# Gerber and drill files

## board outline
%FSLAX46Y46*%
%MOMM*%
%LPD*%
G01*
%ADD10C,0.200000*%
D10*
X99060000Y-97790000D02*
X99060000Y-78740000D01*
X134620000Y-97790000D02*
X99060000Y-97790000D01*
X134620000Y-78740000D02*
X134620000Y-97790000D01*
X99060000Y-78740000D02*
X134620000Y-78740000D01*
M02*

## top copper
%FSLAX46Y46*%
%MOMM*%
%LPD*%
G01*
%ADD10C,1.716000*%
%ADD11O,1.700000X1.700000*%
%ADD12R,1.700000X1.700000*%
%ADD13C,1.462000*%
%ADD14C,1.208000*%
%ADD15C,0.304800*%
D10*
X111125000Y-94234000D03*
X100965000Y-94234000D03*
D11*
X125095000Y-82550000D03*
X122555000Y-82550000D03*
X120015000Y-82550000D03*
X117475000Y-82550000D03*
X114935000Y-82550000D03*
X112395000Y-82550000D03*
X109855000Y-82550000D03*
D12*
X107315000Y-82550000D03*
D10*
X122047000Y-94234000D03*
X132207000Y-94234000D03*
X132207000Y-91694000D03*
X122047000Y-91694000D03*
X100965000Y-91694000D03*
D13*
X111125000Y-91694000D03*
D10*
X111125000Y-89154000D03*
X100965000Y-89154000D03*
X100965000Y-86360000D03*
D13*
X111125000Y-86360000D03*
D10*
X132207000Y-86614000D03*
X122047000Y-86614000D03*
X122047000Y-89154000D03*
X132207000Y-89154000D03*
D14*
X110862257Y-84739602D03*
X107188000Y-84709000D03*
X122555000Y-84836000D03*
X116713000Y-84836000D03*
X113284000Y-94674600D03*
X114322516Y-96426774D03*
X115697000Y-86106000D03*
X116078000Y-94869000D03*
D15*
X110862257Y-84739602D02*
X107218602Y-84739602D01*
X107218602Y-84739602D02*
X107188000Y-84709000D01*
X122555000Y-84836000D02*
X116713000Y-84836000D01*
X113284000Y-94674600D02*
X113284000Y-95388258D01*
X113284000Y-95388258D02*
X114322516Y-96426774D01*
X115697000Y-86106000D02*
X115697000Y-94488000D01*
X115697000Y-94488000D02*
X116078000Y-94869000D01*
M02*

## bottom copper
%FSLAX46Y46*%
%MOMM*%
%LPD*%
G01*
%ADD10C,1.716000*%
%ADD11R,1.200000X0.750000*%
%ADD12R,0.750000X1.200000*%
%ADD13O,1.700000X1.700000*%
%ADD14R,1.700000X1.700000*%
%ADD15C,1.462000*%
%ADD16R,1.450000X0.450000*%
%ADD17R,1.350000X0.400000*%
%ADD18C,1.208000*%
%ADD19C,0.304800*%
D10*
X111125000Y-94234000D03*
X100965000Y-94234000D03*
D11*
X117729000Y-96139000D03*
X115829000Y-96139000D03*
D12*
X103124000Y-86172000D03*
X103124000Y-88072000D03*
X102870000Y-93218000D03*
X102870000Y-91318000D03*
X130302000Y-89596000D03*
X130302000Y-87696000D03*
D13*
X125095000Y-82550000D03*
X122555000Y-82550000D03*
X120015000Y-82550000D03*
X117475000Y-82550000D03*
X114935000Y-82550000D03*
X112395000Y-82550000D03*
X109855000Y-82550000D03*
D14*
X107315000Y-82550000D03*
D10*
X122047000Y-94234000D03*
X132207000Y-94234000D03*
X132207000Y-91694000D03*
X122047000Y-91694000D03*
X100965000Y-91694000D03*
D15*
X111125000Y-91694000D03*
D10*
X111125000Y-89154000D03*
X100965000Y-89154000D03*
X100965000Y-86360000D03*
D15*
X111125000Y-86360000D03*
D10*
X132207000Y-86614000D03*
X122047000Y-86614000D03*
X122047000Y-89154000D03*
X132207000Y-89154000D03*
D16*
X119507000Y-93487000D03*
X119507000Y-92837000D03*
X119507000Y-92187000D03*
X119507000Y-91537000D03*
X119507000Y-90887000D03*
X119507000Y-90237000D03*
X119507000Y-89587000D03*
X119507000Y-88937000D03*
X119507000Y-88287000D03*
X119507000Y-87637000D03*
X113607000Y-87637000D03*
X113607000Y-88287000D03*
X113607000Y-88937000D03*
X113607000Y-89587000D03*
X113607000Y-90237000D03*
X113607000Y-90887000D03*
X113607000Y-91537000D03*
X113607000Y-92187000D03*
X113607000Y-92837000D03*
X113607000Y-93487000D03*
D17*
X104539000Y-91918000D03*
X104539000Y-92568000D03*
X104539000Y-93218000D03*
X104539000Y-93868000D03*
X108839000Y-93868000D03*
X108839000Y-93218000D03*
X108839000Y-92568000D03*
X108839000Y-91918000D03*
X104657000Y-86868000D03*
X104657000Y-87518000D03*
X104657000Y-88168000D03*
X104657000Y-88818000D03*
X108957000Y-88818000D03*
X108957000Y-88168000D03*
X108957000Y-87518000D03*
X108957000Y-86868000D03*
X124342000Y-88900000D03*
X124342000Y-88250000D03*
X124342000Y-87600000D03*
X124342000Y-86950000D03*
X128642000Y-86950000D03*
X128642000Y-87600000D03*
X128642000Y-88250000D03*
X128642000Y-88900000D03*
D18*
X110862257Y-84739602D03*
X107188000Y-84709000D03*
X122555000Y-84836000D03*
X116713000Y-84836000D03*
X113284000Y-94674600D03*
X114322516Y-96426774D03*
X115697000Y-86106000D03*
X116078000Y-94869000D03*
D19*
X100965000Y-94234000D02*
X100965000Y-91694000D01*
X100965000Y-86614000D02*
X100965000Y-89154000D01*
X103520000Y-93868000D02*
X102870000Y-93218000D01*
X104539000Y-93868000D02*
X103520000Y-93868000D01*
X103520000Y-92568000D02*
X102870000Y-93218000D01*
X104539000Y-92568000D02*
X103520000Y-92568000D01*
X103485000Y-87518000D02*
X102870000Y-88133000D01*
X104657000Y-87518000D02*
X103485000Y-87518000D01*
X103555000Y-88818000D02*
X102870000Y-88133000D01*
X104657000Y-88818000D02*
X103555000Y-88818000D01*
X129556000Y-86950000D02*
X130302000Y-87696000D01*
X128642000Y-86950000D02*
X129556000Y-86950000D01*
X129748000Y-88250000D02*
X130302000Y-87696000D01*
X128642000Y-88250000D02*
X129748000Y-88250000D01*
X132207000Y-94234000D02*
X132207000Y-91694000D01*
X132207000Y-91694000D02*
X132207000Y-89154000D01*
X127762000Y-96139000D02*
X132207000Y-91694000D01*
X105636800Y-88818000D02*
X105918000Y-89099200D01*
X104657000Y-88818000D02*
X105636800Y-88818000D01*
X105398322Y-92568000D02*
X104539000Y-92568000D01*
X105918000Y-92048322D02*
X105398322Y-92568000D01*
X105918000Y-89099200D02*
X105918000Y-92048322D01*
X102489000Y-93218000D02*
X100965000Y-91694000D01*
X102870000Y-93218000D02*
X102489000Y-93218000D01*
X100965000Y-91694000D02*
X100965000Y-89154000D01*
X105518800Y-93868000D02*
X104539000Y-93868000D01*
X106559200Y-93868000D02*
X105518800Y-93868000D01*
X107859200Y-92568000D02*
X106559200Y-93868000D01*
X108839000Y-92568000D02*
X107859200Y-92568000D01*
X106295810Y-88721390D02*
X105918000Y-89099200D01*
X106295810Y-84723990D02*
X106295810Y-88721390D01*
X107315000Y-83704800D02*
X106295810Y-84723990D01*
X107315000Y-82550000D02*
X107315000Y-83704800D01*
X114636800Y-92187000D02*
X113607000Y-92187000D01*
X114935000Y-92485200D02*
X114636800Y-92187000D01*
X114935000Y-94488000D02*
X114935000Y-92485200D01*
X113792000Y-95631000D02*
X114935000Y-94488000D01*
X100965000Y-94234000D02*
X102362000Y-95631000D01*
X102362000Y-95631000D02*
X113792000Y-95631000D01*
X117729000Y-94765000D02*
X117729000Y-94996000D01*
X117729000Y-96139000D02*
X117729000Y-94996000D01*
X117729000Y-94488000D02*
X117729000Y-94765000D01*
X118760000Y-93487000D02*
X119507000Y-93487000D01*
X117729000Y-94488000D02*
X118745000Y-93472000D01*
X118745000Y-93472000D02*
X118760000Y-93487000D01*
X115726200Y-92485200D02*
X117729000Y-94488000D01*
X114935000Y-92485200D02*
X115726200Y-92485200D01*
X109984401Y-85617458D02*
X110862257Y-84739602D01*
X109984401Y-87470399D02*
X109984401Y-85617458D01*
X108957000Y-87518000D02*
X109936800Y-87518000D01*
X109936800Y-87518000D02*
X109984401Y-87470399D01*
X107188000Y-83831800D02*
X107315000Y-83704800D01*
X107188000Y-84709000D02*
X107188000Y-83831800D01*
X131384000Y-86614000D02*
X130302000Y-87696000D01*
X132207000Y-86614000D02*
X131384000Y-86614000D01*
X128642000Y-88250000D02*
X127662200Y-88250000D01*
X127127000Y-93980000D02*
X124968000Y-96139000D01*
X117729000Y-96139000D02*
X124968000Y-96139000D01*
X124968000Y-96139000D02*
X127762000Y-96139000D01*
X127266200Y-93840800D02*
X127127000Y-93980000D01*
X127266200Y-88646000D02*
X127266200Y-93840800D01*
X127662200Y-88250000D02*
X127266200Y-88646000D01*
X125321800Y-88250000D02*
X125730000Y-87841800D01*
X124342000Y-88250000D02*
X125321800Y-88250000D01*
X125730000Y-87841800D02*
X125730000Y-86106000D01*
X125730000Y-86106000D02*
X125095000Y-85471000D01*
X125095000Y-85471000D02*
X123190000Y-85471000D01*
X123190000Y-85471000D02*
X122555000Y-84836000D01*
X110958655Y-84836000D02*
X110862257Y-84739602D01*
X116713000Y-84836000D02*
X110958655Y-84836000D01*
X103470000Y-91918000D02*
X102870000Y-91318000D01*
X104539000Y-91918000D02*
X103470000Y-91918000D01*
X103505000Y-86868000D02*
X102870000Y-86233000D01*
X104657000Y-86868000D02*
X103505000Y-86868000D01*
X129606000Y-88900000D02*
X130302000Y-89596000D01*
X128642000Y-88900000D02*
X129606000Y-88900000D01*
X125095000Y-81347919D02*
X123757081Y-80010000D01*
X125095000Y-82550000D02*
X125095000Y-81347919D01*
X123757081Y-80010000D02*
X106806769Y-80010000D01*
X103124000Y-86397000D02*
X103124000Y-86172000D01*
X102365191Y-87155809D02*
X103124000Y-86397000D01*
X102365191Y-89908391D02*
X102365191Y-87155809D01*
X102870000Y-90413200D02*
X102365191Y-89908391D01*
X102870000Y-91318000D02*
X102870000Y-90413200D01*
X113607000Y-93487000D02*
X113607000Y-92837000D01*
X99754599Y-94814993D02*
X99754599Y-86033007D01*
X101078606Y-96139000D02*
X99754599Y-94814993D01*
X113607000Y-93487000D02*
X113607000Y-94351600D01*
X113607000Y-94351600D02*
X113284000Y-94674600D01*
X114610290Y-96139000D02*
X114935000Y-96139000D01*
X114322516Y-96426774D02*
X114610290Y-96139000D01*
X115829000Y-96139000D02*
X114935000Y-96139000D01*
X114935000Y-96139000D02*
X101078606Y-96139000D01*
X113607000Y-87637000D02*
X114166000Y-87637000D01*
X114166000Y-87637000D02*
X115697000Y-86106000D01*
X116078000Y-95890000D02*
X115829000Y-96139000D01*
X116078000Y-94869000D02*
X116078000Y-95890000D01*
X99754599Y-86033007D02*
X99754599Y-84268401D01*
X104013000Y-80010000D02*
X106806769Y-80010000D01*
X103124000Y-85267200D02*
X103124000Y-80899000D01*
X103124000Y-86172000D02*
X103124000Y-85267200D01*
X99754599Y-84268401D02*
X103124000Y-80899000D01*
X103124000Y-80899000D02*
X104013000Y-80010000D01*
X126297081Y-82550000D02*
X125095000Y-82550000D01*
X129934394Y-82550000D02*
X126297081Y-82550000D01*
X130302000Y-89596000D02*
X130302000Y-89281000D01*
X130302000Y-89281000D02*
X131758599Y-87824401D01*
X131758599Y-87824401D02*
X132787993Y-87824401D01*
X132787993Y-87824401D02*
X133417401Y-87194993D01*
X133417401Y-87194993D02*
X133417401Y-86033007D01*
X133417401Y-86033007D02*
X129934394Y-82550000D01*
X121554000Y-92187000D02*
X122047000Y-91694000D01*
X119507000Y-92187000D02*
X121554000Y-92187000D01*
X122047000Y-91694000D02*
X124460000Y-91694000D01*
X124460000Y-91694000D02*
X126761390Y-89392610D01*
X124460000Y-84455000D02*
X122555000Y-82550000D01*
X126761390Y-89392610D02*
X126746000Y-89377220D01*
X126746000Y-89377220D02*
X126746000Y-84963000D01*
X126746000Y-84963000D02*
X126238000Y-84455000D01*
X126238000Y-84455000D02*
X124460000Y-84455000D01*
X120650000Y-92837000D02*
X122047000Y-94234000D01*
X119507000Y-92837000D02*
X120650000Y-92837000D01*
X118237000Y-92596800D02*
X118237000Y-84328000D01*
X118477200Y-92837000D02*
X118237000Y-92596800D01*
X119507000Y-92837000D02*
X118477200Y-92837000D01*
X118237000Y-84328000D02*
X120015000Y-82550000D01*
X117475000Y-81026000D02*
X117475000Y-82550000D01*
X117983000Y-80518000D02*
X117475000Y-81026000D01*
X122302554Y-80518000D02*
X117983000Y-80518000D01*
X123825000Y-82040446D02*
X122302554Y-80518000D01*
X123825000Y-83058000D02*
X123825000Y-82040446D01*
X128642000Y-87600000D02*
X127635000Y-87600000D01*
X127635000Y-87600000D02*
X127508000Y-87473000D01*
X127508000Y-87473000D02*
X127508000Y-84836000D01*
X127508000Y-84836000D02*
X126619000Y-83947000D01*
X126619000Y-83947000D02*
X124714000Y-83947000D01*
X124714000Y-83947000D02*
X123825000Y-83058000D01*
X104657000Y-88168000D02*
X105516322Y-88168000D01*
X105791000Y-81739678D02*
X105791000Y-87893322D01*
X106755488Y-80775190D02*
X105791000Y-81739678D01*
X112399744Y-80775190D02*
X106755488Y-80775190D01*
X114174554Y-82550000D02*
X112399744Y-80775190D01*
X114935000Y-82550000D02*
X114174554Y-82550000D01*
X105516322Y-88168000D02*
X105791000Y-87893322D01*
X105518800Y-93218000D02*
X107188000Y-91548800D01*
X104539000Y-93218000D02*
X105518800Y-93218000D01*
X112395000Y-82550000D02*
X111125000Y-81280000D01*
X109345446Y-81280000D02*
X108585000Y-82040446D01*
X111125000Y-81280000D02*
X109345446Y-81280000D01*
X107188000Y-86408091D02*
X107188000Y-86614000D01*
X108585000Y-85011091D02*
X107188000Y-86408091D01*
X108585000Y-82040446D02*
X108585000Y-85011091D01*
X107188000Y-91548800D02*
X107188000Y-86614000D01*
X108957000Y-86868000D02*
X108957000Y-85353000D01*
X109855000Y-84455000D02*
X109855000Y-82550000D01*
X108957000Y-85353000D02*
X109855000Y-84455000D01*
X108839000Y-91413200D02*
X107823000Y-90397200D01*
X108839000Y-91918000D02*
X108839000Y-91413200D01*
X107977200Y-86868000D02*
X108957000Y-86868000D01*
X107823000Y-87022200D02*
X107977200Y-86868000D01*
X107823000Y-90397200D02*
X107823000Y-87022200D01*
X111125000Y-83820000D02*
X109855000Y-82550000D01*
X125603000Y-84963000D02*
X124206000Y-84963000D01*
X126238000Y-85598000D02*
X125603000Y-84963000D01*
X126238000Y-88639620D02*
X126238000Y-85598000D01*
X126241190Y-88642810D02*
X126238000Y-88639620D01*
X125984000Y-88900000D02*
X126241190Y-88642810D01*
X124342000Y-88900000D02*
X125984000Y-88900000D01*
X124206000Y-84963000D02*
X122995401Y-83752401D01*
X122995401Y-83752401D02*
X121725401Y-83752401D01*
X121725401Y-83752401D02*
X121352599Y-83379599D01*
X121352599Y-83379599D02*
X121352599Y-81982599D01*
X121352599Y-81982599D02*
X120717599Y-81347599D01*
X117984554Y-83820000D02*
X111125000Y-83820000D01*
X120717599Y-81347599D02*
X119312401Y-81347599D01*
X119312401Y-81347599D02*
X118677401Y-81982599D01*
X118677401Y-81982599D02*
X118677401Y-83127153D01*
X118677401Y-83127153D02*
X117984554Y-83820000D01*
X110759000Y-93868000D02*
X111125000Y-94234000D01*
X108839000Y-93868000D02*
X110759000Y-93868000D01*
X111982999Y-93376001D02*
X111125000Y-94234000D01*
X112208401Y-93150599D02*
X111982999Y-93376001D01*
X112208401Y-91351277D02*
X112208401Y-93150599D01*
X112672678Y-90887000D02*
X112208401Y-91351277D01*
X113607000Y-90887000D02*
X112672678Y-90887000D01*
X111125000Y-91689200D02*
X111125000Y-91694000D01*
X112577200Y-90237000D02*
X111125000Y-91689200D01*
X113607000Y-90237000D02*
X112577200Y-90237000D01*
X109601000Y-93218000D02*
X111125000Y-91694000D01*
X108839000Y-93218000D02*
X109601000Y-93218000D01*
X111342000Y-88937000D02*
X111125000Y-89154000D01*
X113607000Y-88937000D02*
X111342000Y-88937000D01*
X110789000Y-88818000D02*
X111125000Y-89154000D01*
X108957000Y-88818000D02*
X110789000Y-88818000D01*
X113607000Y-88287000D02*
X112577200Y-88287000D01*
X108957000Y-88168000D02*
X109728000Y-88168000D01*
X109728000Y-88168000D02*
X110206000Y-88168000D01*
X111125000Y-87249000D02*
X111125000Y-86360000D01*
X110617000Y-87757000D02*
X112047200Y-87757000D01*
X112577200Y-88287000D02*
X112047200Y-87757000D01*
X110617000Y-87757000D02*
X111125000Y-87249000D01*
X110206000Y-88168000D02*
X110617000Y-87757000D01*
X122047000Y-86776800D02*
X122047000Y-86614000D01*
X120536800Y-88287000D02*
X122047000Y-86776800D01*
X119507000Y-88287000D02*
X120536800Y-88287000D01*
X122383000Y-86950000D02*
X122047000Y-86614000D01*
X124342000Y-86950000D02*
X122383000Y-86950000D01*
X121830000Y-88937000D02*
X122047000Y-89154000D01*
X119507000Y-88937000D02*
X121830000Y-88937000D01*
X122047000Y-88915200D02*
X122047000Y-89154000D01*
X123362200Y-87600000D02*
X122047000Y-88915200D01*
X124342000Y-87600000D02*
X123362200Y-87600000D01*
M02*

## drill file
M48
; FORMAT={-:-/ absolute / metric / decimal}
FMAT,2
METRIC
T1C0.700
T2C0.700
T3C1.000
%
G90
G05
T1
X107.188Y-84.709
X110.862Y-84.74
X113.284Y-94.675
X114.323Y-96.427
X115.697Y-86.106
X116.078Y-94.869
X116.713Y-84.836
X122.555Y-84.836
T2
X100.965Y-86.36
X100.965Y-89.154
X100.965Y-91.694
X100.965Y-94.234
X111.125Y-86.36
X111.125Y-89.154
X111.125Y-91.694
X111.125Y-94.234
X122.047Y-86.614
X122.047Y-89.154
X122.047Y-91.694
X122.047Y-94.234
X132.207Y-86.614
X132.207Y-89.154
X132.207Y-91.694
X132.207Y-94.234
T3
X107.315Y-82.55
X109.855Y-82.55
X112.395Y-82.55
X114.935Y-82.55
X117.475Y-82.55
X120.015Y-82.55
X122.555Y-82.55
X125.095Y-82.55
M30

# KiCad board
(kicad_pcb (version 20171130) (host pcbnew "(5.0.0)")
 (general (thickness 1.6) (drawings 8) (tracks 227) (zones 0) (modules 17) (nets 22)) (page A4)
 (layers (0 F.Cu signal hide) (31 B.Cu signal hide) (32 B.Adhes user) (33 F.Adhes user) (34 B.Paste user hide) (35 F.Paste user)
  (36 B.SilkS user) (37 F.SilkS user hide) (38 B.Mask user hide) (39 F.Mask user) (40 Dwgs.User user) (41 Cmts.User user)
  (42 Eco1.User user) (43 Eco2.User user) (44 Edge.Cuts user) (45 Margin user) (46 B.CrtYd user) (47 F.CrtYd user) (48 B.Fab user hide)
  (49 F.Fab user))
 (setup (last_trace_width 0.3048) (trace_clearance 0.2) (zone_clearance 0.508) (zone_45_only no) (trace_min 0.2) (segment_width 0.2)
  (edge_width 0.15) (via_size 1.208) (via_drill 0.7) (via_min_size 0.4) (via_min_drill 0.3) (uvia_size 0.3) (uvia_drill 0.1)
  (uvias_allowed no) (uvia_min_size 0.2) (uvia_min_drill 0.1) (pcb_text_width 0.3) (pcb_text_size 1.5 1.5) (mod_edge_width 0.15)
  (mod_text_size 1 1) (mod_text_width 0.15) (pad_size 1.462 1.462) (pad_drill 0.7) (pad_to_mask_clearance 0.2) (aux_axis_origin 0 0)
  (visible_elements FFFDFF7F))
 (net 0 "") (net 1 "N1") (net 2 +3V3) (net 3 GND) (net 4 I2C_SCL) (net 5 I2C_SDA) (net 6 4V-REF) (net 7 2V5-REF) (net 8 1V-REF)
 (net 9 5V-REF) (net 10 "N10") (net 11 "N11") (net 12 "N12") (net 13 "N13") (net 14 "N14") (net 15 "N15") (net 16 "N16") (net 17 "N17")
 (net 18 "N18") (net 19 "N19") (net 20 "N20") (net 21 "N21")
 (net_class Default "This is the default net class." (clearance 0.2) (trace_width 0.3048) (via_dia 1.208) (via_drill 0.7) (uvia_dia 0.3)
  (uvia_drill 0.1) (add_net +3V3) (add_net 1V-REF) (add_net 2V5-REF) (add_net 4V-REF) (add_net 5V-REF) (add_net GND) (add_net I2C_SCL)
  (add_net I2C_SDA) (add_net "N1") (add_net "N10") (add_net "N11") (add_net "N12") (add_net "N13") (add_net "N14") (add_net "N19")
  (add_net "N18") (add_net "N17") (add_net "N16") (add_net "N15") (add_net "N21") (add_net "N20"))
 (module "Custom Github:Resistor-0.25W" (layer F.Cu) (at 100.965 94.234)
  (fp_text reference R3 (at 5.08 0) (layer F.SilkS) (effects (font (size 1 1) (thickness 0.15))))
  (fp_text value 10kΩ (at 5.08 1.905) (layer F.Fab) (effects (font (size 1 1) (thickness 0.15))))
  (pad 2 thru_hole circle (at 10.16 0) (size 1.716 1.716) (drill 0.7) (layers *.Cu *.Mask F.SilkS) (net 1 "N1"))
  (pad 1 thru_hole circle (at 0 0) (size 1.716 1.716) (drill 0.7) (layers *.Cu *.Mask F.SilkS) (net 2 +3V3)))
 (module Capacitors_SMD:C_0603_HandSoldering (layer B.Cu) (at 116.779 96.139 180)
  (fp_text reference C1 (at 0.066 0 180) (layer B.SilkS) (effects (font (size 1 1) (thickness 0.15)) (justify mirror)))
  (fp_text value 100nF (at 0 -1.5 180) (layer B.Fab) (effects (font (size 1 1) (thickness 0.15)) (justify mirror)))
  (pad 1 smd rect (at -0.95 0 180) (size 1.2 0.75) (layers B.Cu B.Paste B.Mask) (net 2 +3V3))
  (pad 2 smd rect (at 0.95 0 180) (size 1.2 0.75) (layers B.Cu B.Paste B.Mask) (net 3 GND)))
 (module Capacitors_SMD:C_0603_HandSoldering (layer B.Cu) (at 103.124 87.122 90)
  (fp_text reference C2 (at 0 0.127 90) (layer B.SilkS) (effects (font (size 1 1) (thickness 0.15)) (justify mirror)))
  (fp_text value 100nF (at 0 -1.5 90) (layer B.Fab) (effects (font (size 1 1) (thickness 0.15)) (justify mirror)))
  (pad 2 smd rect (at 0.95 0 90) (size 1.2 0.75) (layers B.Cu B.Paste B.Mask) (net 3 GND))
  (pad 1 smd rect (at -0.95 0 90) (size 1.2 0.75) (layers B.Cu B.Paste B.Mask) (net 2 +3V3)))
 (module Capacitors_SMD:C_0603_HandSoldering (layer B.Cu) (at 102.87 92.268 90)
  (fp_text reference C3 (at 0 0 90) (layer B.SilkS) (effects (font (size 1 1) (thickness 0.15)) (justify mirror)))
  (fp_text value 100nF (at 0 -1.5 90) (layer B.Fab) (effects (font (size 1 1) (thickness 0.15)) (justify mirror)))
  (pad 1 smd rect (at -0.95 0 90) (size 1.2 0.75) (layers B.Cu B.Paste B.Mask) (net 2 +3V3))
  (pad 2 smd rect (at 0.95 0 90) (size 1.2 0.75) (layers B.Cu B.Paste B.Mask) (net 3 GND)))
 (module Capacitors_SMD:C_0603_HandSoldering (layer B.Cu) (at 130.302 88.646 270)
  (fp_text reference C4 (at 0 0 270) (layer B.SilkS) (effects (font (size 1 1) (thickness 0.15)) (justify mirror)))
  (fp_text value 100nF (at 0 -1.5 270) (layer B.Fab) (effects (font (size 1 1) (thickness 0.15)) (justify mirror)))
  (pad 2 smd rect (at 0.95 0 270) (size 1.2 0.75) (layers B.Cu B.Paste B.Mask) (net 3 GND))
  (pad 1 smd rect (at -0.95 0 270) (size 1.2 0.75) (layers B.Cu B.Paste B.Mask) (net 2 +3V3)))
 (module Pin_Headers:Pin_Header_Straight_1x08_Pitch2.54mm (layer F.Cu) (at 107.315 82.55 90)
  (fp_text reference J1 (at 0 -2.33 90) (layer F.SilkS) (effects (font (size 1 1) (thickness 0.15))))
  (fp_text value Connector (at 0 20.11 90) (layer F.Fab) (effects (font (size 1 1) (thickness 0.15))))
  (pad 8 thru_hole oval (at 0 17.78 90) (size 1.7 1.7) (drill 1) (layers *.Cu *.Mask) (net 3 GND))
  (pad 7 thru_hole oval (at 0 15.24 90) (size 1.7 1.7) (drill 1) (layers *.Cu *.Mask) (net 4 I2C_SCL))
  (pad 6 thru_hole oval (at 0 12.7 90) (size 1.7 1.7) (drill 1) (layers *.Cu *.Mask) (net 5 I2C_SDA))
  (pad 5 thru_hole oval (at 0 10.16 90) (size 1.7 1.7) (drill 1) (layers *.Cu *.Mask) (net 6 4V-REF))
  (pad 4 thru_hole oval (at 0 7.62 90) (size 1.7 1.7) (drill 1) (layers *.Cu *.Mask) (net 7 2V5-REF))
  (pad 3 thru_hole oval (at 0 5.08 90) (size 1.7 1.7) (drill 1) (layers *.Cu *.Mask) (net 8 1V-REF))
  (pad 2 thru_hole oval (at 0 2.54 90) (size 1.7 1.7) (drill 1) (layers *.Cu *.Mask) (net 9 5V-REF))
  (pad 1 thru_hole rect (at 0 0 90) (size 1.7 1.7) (drill 1) (layers *.Cu *.Mask) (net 2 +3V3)))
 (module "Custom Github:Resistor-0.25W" (layer F.Cu) (at 132.207 94.234 180)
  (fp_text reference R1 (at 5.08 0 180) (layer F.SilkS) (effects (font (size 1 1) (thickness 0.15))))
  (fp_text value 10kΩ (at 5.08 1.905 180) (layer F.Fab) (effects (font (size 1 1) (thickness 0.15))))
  (pad 2 thru_hole circle (at 10.16 0 180) (size 1.716 1.716) (drill 0.7) (layers *.Cu *.Mask F.SilkS) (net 5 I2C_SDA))
  (pad 1 thru_hole circle (at 0 0 180) (size 1.716 1.716) (drill 0.7) (layers *.Cu *.Mask F.SilkS) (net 2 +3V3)))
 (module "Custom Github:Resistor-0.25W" (layer F.Cu) (at 132.207 91.694 180)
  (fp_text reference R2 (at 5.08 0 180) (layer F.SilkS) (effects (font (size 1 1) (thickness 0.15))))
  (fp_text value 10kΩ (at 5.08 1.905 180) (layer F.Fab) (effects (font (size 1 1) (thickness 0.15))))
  (pad 1 thru_hole circle (at 0 0 180) (size 1.716 1.716) (drill 0.7) (layers *.Cu *.Mask F.SilkS) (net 2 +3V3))
  (pad 2 thru_hole circle (at 10.16 0 180) (size 1.716 1.716) (drill 0.7) (layers *.Cu *.Mask F.SilkS) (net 4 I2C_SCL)))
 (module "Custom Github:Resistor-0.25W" (layer F.Cu) (at 100.965 91.694)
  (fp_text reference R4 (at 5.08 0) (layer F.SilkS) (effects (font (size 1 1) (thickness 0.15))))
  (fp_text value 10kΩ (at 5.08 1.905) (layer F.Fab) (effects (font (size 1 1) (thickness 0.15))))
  (pad 1 thru_hole circle (at 0 0) (size 1.716 1.716) (drill 0.7) (layers *.Cu *.Mask F.SilkS) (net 2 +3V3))
  (pad 2 thru_hole circle (at 10.16 0) (size 1.462 1.462) (drill 0.7) (layers *.Cu *.Mask F.SilkS) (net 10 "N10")))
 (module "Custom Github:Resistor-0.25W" (layer F.Cu) (at 100.965 89.154)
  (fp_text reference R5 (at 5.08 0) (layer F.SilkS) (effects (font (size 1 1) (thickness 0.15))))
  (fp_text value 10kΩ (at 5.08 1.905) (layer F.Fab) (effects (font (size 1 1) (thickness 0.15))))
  (pad 2 thru_hole circle (at 10.16 0) (size 1.716 1.716) (drill 0.7) (layers *.Cu *.Mask F.SilkS) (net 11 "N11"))
  (pad 1 thru_hole circle (at 0 0) (size 1.716 1.716) (drill 0.7) (layers *.Cu *.Mask F.SilkS) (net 2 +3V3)))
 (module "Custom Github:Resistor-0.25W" (layer F.Cu) (at 100.965 86.36)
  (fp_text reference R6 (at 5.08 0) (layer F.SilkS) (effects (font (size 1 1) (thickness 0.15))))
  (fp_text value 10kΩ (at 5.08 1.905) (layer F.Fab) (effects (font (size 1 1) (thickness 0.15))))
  (pad 1 thru_hole circle (at 0 0) (size 1.716 1.716) (drill 0.7) (layers *.Cu *.Mask F.SilkS) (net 2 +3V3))
  (pad 2 thru_hole circle (at 10.16 0) (size 1.462 1.462) (drill 0.7) (layers *.Cu *.Mask F.SilkS) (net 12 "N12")))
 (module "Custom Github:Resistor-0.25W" (layer F.Cu) (at 132.207 86.614 180)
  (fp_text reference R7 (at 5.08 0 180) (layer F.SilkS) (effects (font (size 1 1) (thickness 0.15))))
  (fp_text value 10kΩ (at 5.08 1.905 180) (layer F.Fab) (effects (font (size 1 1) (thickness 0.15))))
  (pad 1 thru_hole circle (at 0 0 180) (size 1.716 1.716) (drill 0.7) (layers *.Cu *.Mask F.SilkS) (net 2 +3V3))
  (pad 2 thru_hole circle (at 10.16 0 180) (size 1.716 1.716) (drill 0.7) (layers *.Cu *.Mask F.SilkS) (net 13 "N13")))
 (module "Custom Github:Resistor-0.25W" (layer F.Cu) (at 132.207 89.154 180)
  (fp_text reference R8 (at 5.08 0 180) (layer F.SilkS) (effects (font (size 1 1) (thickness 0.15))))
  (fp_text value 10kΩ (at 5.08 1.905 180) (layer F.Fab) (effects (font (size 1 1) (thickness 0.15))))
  (pad 2 thru_hole circle (at 10.16 0 180) (size 1.716 1.716) (drill 0.7) (layers *.Cu *.Mask F.SilkS) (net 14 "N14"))
  (pad 1 thru_hole circle (at 0 0 180) (size 1.716 1.716) (drill 0.7) (layers *.Cu *.Mask F.SilkS) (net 2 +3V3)))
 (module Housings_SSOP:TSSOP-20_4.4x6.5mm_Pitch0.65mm (layer B.Cu) (at 116.557 90.562)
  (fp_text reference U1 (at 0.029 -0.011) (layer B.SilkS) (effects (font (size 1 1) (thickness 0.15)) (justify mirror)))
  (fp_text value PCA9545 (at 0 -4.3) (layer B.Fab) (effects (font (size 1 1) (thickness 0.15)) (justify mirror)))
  (pad 20 smd rect (at 2.95 2.925) (size 1.45 0.45) (layers B.Cu B.Paste B.Mask) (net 2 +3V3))
  (pad 19 smd rect (at 2.95 2.275) (size 1.45 0.45) (layers B.Cu B.Paste B.Mask) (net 5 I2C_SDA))
  (pad 18 smd rect (at 2.95 1.625) (size 1.45 0.45) (layers B.Cu B.Paste B.Mask) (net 4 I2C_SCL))
  (pad 17 smd rect (at 2.95 0.975) (size 1.45 0.45) (layers B.Cu B.Paste B.Mask) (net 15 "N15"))
  (pad 16 smd rect (at 2.95 0.325) (size 1.45 0.45) (layers B.Cu B.Paste B.Mask) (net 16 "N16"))
  (pad 15 smd rect (at 2.95 -0.325) (size 1.45 0.45) (layers B.Cu B.Paste B.Mask) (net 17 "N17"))
  (pad 14 smd rect (at 2.95 -0.975) (size 1.45 0.45) (layers B.Cu B.Paste B.Mask) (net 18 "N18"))
  (pad 13 smd rect (at 2.95 -1.625) (size 1.45 0.45) (layers B.Cu B.Paste B.Mask) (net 14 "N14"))
  (pad 12 smd rect (at 2.95 -2.275) (size 1.45 0.45) (layers B.Cu B.Paste B.Mask) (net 13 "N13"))
  (pad 11 smd rect (at 2.95 -2.925) (size 1.45 0.45) (layers B.Cu B.Paste B.Mask) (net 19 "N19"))
  (pad 10 smd rect (at -2.95 -2.925) (size 1.45 0.45) (layers B.Cu B.Paste B.Mask) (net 3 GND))
  (pad 9 smd rect (at -2.95 -2.275) (size 1.45 0.45) (layers B.Cu B.Paste B.Mask) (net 12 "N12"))
  (pad 8 smd rect (at -2.95 -1.625) (size 1.45 0.45) (layers B.Cu B.Paste B.Mask) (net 11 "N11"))
  (pad 7 smd rect (at -2.95 -0.975) (size 1.45 0.45) (layers B.Cu B.Paste B.Mask) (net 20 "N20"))
  (pad 6 smd rect (at -2.95 -0.325) (size 1.45 0.45) (layers B.Cu B.Paste B.Mask) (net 10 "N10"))
  (pad 5 smd rect (at -2.95 0.325) (size 1.45 0.45) (layers B.Cu B.Paste B.Mask) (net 1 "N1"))
  (pad 4 smd rect (at -2.95 0.975) (size 1.45 0.45) (layers B.Cu B.Paste B.Mask) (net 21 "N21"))
  (pad 3 smd rect (at -2.95 1.625) (size 1.45 0.45) (layers B.Cu B.Paste B.Mask) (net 2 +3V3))
  (pad 2 smd rect (at -2.95 2.275) (size 1.45 0.45) (layers B.Cu B.Paste B.Mask) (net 3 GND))
  (pad 1 smd rect (at -2.95 2.925) (size 1.45 0.45) (layers B.Cu B.Paste B.Mask) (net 3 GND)))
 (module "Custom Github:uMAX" (layer B.Cu) (at 106.689 91.918 180)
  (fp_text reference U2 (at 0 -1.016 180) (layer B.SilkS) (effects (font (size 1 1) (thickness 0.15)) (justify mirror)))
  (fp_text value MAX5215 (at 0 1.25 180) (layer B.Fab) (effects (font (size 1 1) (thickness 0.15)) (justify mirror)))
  (pad 8 smd rect (at 2.15 0 180) (size 1.35 0.4) (layers B.Cu B.Paste B.Mask) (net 3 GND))
  (pad 7 smd rect (at 2.15 -0.65 180) (size 1.35 0.4) (layers B.Cu B.Paste B.Mask) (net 2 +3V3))
  (pad 6 smd rect (at 2.15 -1.3 180) (size 1.35 0.4) (layers B.Cu B.Paste B.Mask) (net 8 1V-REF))
  (pad 5 smd rect (at 2.15 -1.95 180) (size 1.35 0.4) (layers B.Cu B.Paste B.Mask) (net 2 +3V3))
  (pad 4 smd rect (at -2.15 -1.95 180) (size 1.35 0.4) (layers B.Cu B.Paste B.Mask) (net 1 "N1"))
  (pad 3 smd rect (at -2.15 -1.3 180) (size 1.35 0.4) (layers B.Cu B.Paste B.Mask) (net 10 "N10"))
  (pad 2 smd rect (at -2.15 -0.65 180) (size 1.35 0.4) (layers B.Cu B.Paste B.Mask) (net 2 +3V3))
  (pad 1 smd rect (at -2.15 0 180) (size 1.35 0.4) (layers B.Cu B.Paste B.Mask) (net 9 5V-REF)))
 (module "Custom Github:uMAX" (layer B.Cu) (at 106.807 86.868 180)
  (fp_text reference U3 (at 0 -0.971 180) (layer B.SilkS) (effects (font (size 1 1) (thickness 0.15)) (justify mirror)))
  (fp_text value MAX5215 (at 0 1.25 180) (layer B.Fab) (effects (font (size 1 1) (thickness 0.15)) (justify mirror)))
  (pad 8 smd rect (at 2.15 0 180) (size 1.35 0.4) (layers B.Cu B.Paste B.Mask) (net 3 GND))
  (pad 7 smd rect (at 2.15 -0.65 180) (size 1.35 0.4) (layers B.Cu B.Paste B.Mask) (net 2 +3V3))
  (pad 6 smd rect (at 2.15 -1.3 180) (size 1.35 0.4) (layers B.Cu B.Paste B.Mask) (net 7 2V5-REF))
  (pad 5 smd rect (at 2.15 -1.95 180) (size 1.35 0.4) (layers B.Cu B.Paste B.Mask) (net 2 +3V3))
  (pad 4 smd rect (at -2.15 -1.95 180) (size 1.35 0.4) (layers B.Cu B.Paste B.Mask) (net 11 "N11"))
  (pad 3 smd rect (at -2.15 -1.3 180) (size 1.35 0.4) (layers B.Cu B.Paste B.Mask) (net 12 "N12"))
  (pad 2 smd rect (at -2.15 -0.65 180) (size 1.35 0.4) (layers B.Cu B.Paste B.Mask) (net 2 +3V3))
  (pad 1 smd rect (at -2.15 0 180) (size 1.35 0.4) (layers B.Cu B.Paste B.Mask) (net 9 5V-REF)))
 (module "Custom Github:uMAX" (layer B.Cu) (at 126.492 88.9)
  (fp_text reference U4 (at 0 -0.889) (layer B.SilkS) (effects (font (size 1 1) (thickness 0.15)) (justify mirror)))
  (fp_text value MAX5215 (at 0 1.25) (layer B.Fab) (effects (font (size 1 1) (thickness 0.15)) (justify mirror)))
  (pad 1 smd rect (at -2.15 0) (size 1.35 0.4) (layers B.Cu B.Paste B.Mask) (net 9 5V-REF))
  (pad 2 smd rect (at -2.15 -0.65) (size 1.35 0.4) (layers B.Cu B.Paste B.Mask) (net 2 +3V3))
  (pad 3 smd rect (at -2.15 -1.3) (size 1.35 0.4) (layers B.Cu B.Paste B.Mask) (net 14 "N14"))
  (pad 4 smd rect (at -2.15 -1.95) (size 1.35 0.4) (layers B.Cu B.Paste B.Mask) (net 13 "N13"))
  (pad 5 smd rect (at 2.15 -1.95) (size 1.35 0.4) (layers B.Cu B.Paste B.Mask) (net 2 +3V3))
  (pad 6 smd rect (at 2.15 -1.3) (size 1.35 0.4) (layers B.Cu B.Paste B.Mask) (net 6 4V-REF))
  (pad 7 smd rect (at 2.15 -0.65) (size 1.35 0.4) (layers B.Cu B.Paste B.Mask) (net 2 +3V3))
  (pad 8 smd rect (at 2.15 0) (size 1.35 0.4) (layers B.Cu B.Paste B.Mask) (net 3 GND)))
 (gr_line (start 99.06 97.79) (end 99.06 78.74) (layer Edge.Cuts) (width 0.2))
 (gr_line (start 134.62 97.79) (end 99.06 97.79) (layer Edge.Cuts) (width 0.2))
 (gr_line (start 134.62 78.74) (end 134.62 97.79) (layer Edge.Cuts) (width 0.2))
 (gr_line (start 99.06 78.74) (end 134.62 78.74) (layer Edge.Cuts) (width 0.2))
 (segment (start 100.965 94.234) (end 100.965 91.694) (width 0.3048) (layer B.Cu) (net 2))
 (segment (start 100.965 86.614) (end 100.965 89.154) (width 0.3048) (layer B.Cu) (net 2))
 (segment (start 103.52 93.868) (end 102.87 93.218) (width 0.3048) (layer B.Cu) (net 2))
 (segment (start 104.539 93.868) (end 103.52 93.868) (width 0.3048) (layer B.Cu) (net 2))
 (segment (start 103.52 92.568) (end 102.87 93.218) (width 0.3048) (layer B.Cu) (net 2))
 (segment (start 104.539 92.568) (end 103.52 92.568) (width 0.3048) (layer B.Cu) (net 2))
 (segment (start 103.485 87.518) (end 102.87 88.133) (width 0.3048) (layer B.Cu) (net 2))
 (segment (start 104.657 87.518) (end 103.485 87.518) (width 0.3048) (layer B.Cu) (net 2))
 (segment (start 103.555 88.818) (end 102.87 88.133) (width 0.3048) (layer B.Cu) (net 2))
 (segment (start 104.657 88.818) (end 103.555 88.818) (width 0.3048) (layer B.Cu) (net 2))
 (segment (start 129.556 86.95) (end 130.302 87.696) (width 0.3048) (layer B.Cu) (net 2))
 (segment (start 128.642 86.95) (end 129.556 86.95) (width 0.3048) (layer B.Cu) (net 2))
 (segment (start 129.748 88.25) (end 130.302 87.696) (width 0.3048) (layer B.Cu) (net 2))
 (segment (start 128.642 88.25) (end 129.748 88.25) (width 0.3048) (layer B.Cu) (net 2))
 (segment (start 132.207 94.234) (end 132.207 91.694) (width 0.3048) (layer B.Cu) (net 2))
 (segment (start 132.207 91.694) (end 132.207 89.154) (width 0.3048) (layer B.Cu) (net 2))
 (segment (start 127.762 96.139) (end 132.207 91.694) (width 0.3048) (layer B.Cu) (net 2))
 (segment (start 105.6368 88.818) (end 105.918 89.0992) (width 0.3048) (layer B.Cu) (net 2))
 (segment (start 104.657 88.818) (end 105.6368 88.818) (width 0.3048) (layer B.Cu) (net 2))
 (segment (start 105.398322 92.568) (end 104.539 92.568) (width 0.3048) (layer B.Cu) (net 2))
 (segment (start 105.918 92.048322) (end 105.398322 92.568) (width 0.3048) (layer B.Cu) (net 2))
 (segment (start 105.918 89.0992) (end 105.918 92.048322) (width 0.3048) (layer B.Cu) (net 2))
 (segment (start 102.489 93.218) (end 100.965 91.694) (width 0.3048) (layer B.Cu) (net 2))
 (segment (start 102.87 93.218) (end 102.489 93.218) (width 0.3048) (layer B.Cu) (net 2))
 (segment (start 100.965 91.694) (end 100.965 89.154) (width 0.3048) (layer B.Cu) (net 2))
 (segment (start 105.5188 93.868) (end 104.539 93.868) (width 0.3048) (layer B.Cu) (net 2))
 (segment (start 106.5592 93.868) (end 105.5188 93.868) (width 0.3048) (layer B.Cu) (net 2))
 (segment (start 107.8592 92.568) (end 106.5592 93.868) (width 0.3048) (layer B.Cu) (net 2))
 (segment (start 108.839 92.568) (end 107.8592 92.568) (width 0.3048) (layer B.Cu) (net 2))
 (segment (start 106.29581 88.72139) (end 105.918 89.0992) (width 0.3048) (layer B.Cu) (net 2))
 (segment (start 106.29581 84.72399) (end 106.29581 88.72139) (width 0.3048) (layer B.Cu) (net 2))
 (segment (start 107.315 83.7048) (end 106.29581 84.72399) (width 0.3048) (layer B.Cu) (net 2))
 (segment (start 107.315 82.55) (end 107.315 83.7048) (width 0.3048) (layer B.Cu) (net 2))
 (segment (start 114.6368 92.187) (end 113.607 92.187) (width 0.3048) (layer B.Cu) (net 2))
 (segment (start 114.935 92.4852) (end 114.6368 92.187) (width 0.3048) (layer B.Cu) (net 2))
 (segment (start 114.935 94.488) (end 114.935 92.4852) (width 0.3048) (layer B.Cu) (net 2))
 (segment (start 113.792 95.631) (end 114.935 94.488) (width 0.3048) (layer B.Cu) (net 2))
 (segment (start 100.965 94.234) (end 102.362 95.631) (width 0.3048) (layer B.Cu) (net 2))
 (segment (start 102.362 95.631) (end 113.792 95.631) (width 0.3048) (layer B.Cu) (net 2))
 (segment (start 117.729 94.765) (end 117.729 94.996) (width 0.3048) (layer B.Cu) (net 2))
 (segment (start 117.729 96.139) (end 117.729 94.996) (width 0.3048) (layer B.Cu) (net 2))
 (segment (start 117.729 94.488) (end 117.729 94.765) (width 0.3048) (layer B.Cu) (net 2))
 (segment (start 118.76 93.487) (end 119.507 93.487) (width 0.3048) (layer B.Cu) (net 2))
 (segment (start 117.729 94.488) (end 118.745 93.472) (width 0.3048) (layer B.Cu) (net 2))
 (segment (start 118.745 93.472) (end 118.76 93.487) (width 0.3048) (layer B.Cu) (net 2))
 (segment (start 115.7262 92.4852) (end 117.729 94.488) (width 0.3048) (layer B.Cu) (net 2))
 (segment (start 114.935 92.4852) (end 115.7262 92.4852) (width 0.3048) (layer B.Cu) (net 2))
 (via (at 110.862257 84.739602) (size 1.208) (drill 0.7) (layers F.Cu B.Cu) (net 2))
 (segment (start 109.984401 85.617458) (end 110.862257 84.739602) (width 0.3048) (layer B.Cu) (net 2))
 (segment (start 109.984401 87.470399) (end 109.984401 85.617458) (width 0.3048) (layer B.Cu) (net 2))
 (segment (start 108.957 87.518) (end 109.9368 87.518) (width 0.3048) (layer B.Cu) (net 2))
 (segment (start 109.9368 87.518) (end 109.984401 87.470399) (width 0.3048) (layer B.Cu) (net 2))
 (via (at 107.188 84.709) (size 1.208) (drill 0.7) (layers F.Cu B.Cu) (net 2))
 (segment (start 110.862257 84.739602) (end 107.218602 84.739602) (width 0.3048) (layer F.Cu) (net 2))
 (segment (start 107.218602 84.739602) (end 107.188 84.709) (width 0.3048) (layer F.Cu) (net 2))
 (segment (start 107.188 83.8318) (end 107.315 83.7048) (width 0.3048) (layer B.Cu) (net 2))
 (segment (start 107.188 84.709) (end 107.188 83.8318) (width 0.3048) (layer B.Cu) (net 2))
 (segment (start 131.384 86.614) (end 130.302 87.696) (width 0.3048) (layer B.Cu) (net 2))
 (segment (start 132.207 86.614) (end 131.384 86.614) (width 0.3048) (layer B.Cu) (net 2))
 (segment (start 128.642 88.25) (end 127.6622 88.25) (width 0.3048) (layer B.Cu) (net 2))
 (segment (start 127.127 93.98) (end 124.968 96.139) (width 0.3048) (layer B.Cu) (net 2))
 (segment (start 117.729 96.139) (end 124.968 96.139) (width 0.3048) (layer B.Cu) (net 2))
 (segment (start 124.968 96.139) (end 127.762 96.139) (width 0.3048) (layer B.Cu) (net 2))
 (segment (start 127.2662 93.8408) (end 127.127 93.98) (width 0.3048) (layer B.Cu) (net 2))
 (segment (start 127.2662 88.646) (end 127.2662 93.8408) (width 0.3048) (layer B.Cu) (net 2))
 (segment (start 127.6622 88.25) (end 127.2662 88.646) (width 0.3048) (layer B.Cu) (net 2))
 (segment (start 125.3218 88.25) (end 125.73 87.8418) (width 0.3048) (layer B.Cu) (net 2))
 (segment (start 124.342 88.25) (end 125.3218 88.25) (width 0.3048) (layer B.Cu) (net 2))
 (segment (start 125.73 87.8418) (end 125.73 86.106) (width 0.3048) (layer B.Cu) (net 2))
 (segment (start 125.73 86.106) (end 125.095 85.471) (width 0.3048) (layer B.Cu) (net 2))
 (via (at 122.555 84.836) (size 1.208) (drill 0.7) (layers F.Cu B.Cu) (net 2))
 (segment (start 125.095 85.471) (end 123.19 85.471) (width 0.3048) (layer B.Cu) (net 2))
 (segment (start 123.19 85.471) (end 122.555 84.836) (width 0.3048) (layer B.Cu) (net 2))
 (via (at 116.713 84.836) (size 1.208) (drill 0.7) (layers F.Cu B.Cu) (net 2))
 (segment (start 122.555 84.836) (end 116.713 84.836) (width 0.3048) (layer F.Cu) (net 2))
 (segment (start 110.958655 84.836) (end 110.862257 84.739602) (width 0.3048) (layer B.Cu) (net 2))
 (segment (start 116.713 84.836) (end 110.958655 84.836) (width 0.3048) (layer B.Cu) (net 2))
 (segment (start 103.47 91.918) (end 102.87 91.318) (width 0.3048) (layer B.Cu) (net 3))
 (segment (start 104.539 91.918) (end 103.47 91.918) (width 0.3048) (layer B.Cu) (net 3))
 (segment (start 103.505 86.868) (end 102.87 86.233) (width 0.3048) (layer B.Cu) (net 3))
 (segment (start 104.657 86.868) (end 103.505 86.868) (width 0.3048) (layer B.Cu) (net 3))
 (segment (start 129.606 88.9) (end 130.302 89.596) (width 0.3048) (layer B.Cu) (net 3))
 (segment (start 128.642 88.9) (end 129.606 88.9) (width 0.3048) (layer B.Cu) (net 3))
 (segment (start 125.095 81.347919) (end 123.757081 80.01) (width 0.3048) (layer B.Cu) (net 3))
 (segment (start 125.095 82.55) (end 125.095 81.347919) (width 0.3048) (layer B.Cu) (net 3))
 (segment (start 123.757081 80.01) (end 106.806769 80.01) (width 0.3048) (layer B.Cu) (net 3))
 (segment (start 103.124 86.397) (end 103.124 86.172) (width 0.3048) (layer B.Cu) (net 3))
 (segment (start 102.365191 87.155809) (end 103.124 86.397) (width 0.3048) (layer B.Cu) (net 3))
 (segment (start 102.365191 89.908391) (end 102.365191 87.155809) (width 0.3048) (layer B.Cu) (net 3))
 (segment (start 102.87 90.4132) (end 102.365191 89.908391) (width 0.3048) (layer B.Cu) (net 3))
 (segment (start 102.87 91.318) (end 102.87 90.4132) (width 0.3048) (layer B.Cu) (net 3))
 (segment (start 113.607 93.487) (end 113.607 92.837) (width 0.3048) (layer B.Cu) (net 3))
 (segment (start 99.754599 94.814993) (end 99.754599 86.033007) (width 0.3048) (layer B.Cu) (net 3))
 (segment (start 101.078606 96.139) (end 99.754599 94.814993) (width 0.3048) (layer B.Cu) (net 3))
 (via (at 113.284 94.6746) (size 1.208) (drill 0.7) (layers F.Cu B.Cu) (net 3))
 (segment (start 113.607 93.487) (end 113.607 94.3516) (width 0.3048) (layer B.Cu) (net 3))
 (segment (start 113.607 94.3516) (end 113.284 94.6746) (width 0.3048) (layer B.Cu) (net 3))
 (via (at 114.322516 96.426774) (size 1.208) (drill 0.7) (layers F.Cu B.Cu) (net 3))
 (segment (start 113.284 94.6746) (end 113.284 95.388258) (width 0.3048) (layer F.Cu) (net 3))
 (segment (start 113.284 95.388258) (end 114.322516 96.426774) (width 0.3048) (layer F.Cu) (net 3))
 (segment (start 114.61029 96.139) (end 114.935 96.139) (width 0.3048) (layer B.Cu) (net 3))
 (segment (start 114.322516 96.426774) (end 114.61029 96.139) (width 0.3048) (layer B.Cu) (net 3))
 (segment (start 115.829 96.139) (end 114.935 96.139) (width 0.3048) (layer B.Cu) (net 3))
 (segment (start 114.935 96.139) (end 101.078606 96.139) (width 0.3048) (layer B.Cu) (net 3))
 (via (at 115.697 86.106) (size 1.208) (drill 0.7) (layers F.Cu B.Cu) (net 3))
 (segment (start 113.607 87.637) (end 114.166 87.637) (width 0.3048) (layer B.Cu) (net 3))
 (segment (start 114.166 87.637) (end 115.697 86.106) (width 0.3048) (layer B.Cu) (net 3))
 (via (at 116.078 94.869) (size 1.208) (drill 0.7) (layers F.Cu B.Cu) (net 3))
 (segment (start 115.697 86.106) (end 115.697 94.488) (width 0.3048) (layer F.Cu) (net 3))
 (segment (start 115.697 94.488) (end 116.078 94.869) (width 0.3048) (layer F.Cu) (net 3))
 (segment (start 116.078 95.89) (end 115.829 96.139) (width 0.3048) (layer B.Cu) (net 3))
 (segment (start 116.078 94.869) (end 116.078 95.89) (width 0.3048) (layer B.Cu) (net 3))
 (segment (start 99.754599 86.033007) (end 99.754599 84.268401) (width 0.3048) (layer B.Cu) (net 3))
 (segment (start 104.013 80.01) (end 106.806769 80.01) (width 0.3048) (layer B.Cu) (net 3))
 (segment (start 103.124 85.2672) (end 103.124 80.899) (width 0.3048) (layer B.Cu) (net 3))
 (segment (start 103.124 86.172) (end 103.124 85.2672) (width 0.3048) (layer B.Cu) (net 3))
 (segment (start 99.754599 84.268401) (end 103.124 80.899) (width 0.3048) (layer B.Cu) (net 3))
 (segment (start 103.124 80.899) (end 104.013 80.01) (width 0.3048) (layer B.Cu) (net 3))
 (segment (start 126.297081 82.55) (end 125.095 82.55) (width 0.3048) (layer B.Cu) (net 3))
 (segment (start 129.934394 82.55) (end 126.297081 82.55) (width 0.3048) (layer B.Cu) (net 3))
 (segment (start 130.302 89.596) (end 130.302 89.281) (width 0.3048) (layer B.Cu) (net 3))
 (segment (start 130.302 89.281) (end 131.758599 87.824401) (width 0.3048) (layer B.Cu) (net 3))
 (segment (start 131.758599 87.824401) (end 132.787993 87.824401) (width 0.3048) (layer B.Cu) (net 3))
 (segment (start 132.787993 87.824401) (end 133.417401 87.194993) (width 0.3048) (layer B.Cu) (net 3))
 (segment (start 133.417401 87.194993) (end 133.417401 86.033007) (width 0.3048) (layer B.Cu) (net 3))
 (segment (start 133.417401 86.033007) (end 129.934394 82.55) (width 0.3048) (layer B.Cu) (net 3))
 (segment (start 121.554 92.187) (end 122.047 91.694) (width 0.3048) (layer B.Cu) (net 4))
 (segment (start 119.507 92.187) (end 121.554 92.187) (width 0.3048) (layer B.Cu) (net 4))
 (segment (start 122.047 91.694) (end 124.46 91.694) (width 0.3048) (layer B.Cu) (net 4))
 (segment (start 124.46 91.694) (end 126.76139 89.39261) (width 0.3048) (layer B.Cu) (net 4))
 (segment (start 124.46 84.455) (end 122.555 82.55) (width 0.3048) (layer B.Cu) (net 4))
 (segment (start 126.76139 89.39261) (end 126.746 89.37722) (width 0.3048) (layer B.Cu) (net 4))
 (segment (start 126.746 89.37722) (end 126.746 84.963) (width 0.3048) (layer B.Cu) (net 4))
 (segment (start 126.746 84.963) (end 126.238 84.455) (width 0.3048) (layer B.Cu) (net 4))
 (segment (start 126.238 84.455) (end 124.46 84.455) (width 0.3048) (layer B.Cu) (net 4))
 (segment (start 120.65 92.837) (end 122.047 94.234) (width 0.3048) (layer B.Cu) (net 5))
 (segment (start 119.507 92.837) (end 120.65 92.837) (width 0.3048) (layer B.Cu) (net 5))
 (segment (start 118.237 92.5968) (end 118.237 84.328) (width 0.3048) (layer B.Cu) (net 5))
 (segment (start 118.4772 92.837) (end 118.237 92.5968) (width 0.3048) (layer B.Cu) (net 5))
 (segment (start 119.507 92.837) (end 118.4772 92.837) (width 0.3048) (layer B.Cu) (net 5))
 (segment (start 118.237 84.328) (end 120.015 82.55) (width 0.3048) (layer B.Cu) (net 5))
 (segment (start 117.475 81.026) (end 117.475 82.55) (width 0.3048) (layer B.Cu) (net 6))
 (segment (start 117.983 80.518) (end 117.475 81.026) (width 0.3048) (layer B.Cu) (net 6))
 (segment (start 122.302554 80.518) (end 117.983 80.518) (width 0.3048) (layer B.Cu) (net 6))
 (segment (start 123.825 82.040446) (end 122.302554 80.518) (width 0.3048) (layer B.Cu) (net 6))
 (segment (start 123.825 83.058) (end 123.825 82.040446) (width 0.3048) (layer B.Cu) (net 6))
 (segment (start 128.642 87.6) (end 127.635 87.6) (width 0.3048) (layer B.Cu) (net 6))
 (segment (start 127.635 87.6) (end 127.508 87.473) (width 0.3048) (layer B.Cu) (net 6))
 (segment (start 127.508 87.473) (end 127.508 84.836) (width 0.3048) (layer B.Cu) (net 6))
 (segment (start 127.508 84.836) (end 126.619 83.947) (width 0.3048) (layer B.Cu) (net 6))
 (segment (start 126.619 83.947) (end 124.714 83.947) (width 0.3048) (layer B.Cu) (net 6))
 (segment (start 124.714 83.947) (end 123.825 83.058) (width 0.3048) (layer B.Cu) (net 6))
 (segment (start 104.657 88.168) (end 105.516322 88.168) (width 0.3048) (layer B.Cu) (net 7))
 (segment (start 105.791 81.739678) (end 105.791 87.893322) (width 0.3048) (layer B.Cu) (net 7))
 (segment (start 106.755488 80.77519) (end 105.791 81.739678) (width 0.3048) (layer B.Cu) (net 7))
 (segment (start 112.399744 80.77519) (end 106.755488 80.77519) (width 0.3048) (layer B.Cu) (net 7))
 (segment (start 114.174554 82.55) (end 112.399744 80.77519) (width 0.3048) (layer B.Cu) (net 7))
 (segment (start 114.935 82.55) (end 114.174554 82.55) (width 0.3048) (layer B.Cu) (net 7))
 (segment (start 105.516322 88.168) (end 105.791 87.893322) (width 0.3048) (layer B.Cu) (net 7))
 (segment (start 105.5188 93.218) (end 107.188 91.5488) (width 0.3048) (layer B.Cu) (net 8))
 (segment (start 104.539 93.218) (end 105.5188 93.218) (width 0.3048) (layer B.Cu) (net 8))
 (segment (start 112.395 82.55) (end 111.125 81.28) (width 0.3048) (layer B.Cu) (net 8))
 (segment (start 109.345446 81.28) (end 108.585 82.040446) (width 0.3048) (layer B.Cu) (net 8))
 (segment (start 111.125 81.28) (end 109.345446 81.28) (width 0.3048) (layer B.Cu) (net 8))
 (segment (start 107.188 86.408091) (end 107.188 86.614) (width 0.3048) (layer B.Cu) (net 8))
 (segment (start 108.585 85.011091) (end 107.188 86.408091) (width 0.3048) (layer B.Cu) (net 8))
 (segment (start 108.585 82.040446) (end 108.585 85.011091) (width 0.3048) (layer B.Cu) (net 8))
 (segment (start 107.188 91.5488) (end 107.188 86.614) (width 0.3048) (layer B.Cu) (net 8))
 (segment (start 108.957 86.868) (end 108.957 85.353) (width 0.3048) (layer B.Cu) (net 9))
 (segment (start 109.855 84.455) (end 109.855 82.55) (width 0.3048) (layer B.Cu) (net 9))
 (segment (start 108.957 85.353) (end 109.855 84.455) (width 0.3048) (layer B.Cu) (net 9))
 (segment (start 108.839 91.4132) (end 107.823 90.3972) (width 0.3048) (layer B.Cu) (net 9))
 (segment (start 108.839 91.918) (end 108.839 91.4132) (width 0.3048) (layer B.Cu) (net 9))
 (segment (start 107.9772 86.868) (end 108.957 86.868) (width 0.3048) (layer B.Cu) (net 9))
 (segment (start 107.823 87.0222) (end 107.9772 86.868) (width 0.3048) (layer B.Cu) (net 9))
 (segment (start 107.823 90.3972) (end 107.823 87.0222) (width 0.3048) (layer B.Cu) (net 9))
 (segment (start 111.125 83.82) (end 109.855 82.55) (width 0.3048) (layer B.Cu) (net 9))
 (segment (start 125.603 84.963) (end 124.206 84.963) (width 0.3048) (layer B.Cu) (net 9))
 (segment (start 126.238 85.598) (end 125.603 84.963) (width 0.3048) (layer B.Cu) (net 9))
 (segment (start 126.238 88.63962) (end 126.238 85.598) (width 0.3048) (layer B.Cu) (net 9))
 (segment (start 126.24119 88.64281) (end 126.238 88.63962) (width 0.3048) (layer B.Cu) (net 9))
 (segment (start 125.984 88.9) (end 126.24119 88.64281) (width 0.3048) (layer B.Cu) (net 9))
 (segment (start 124.342 88.9) (end 125.984 88.9) (width 0.3048) (layer B.Cu) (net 9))
 (segment (start 124.206 84.963) (end 122.995401 83.752401) (width 0.3048) (layer B.Cu) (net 9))
 (segment (start 122.995401 83.752401) (end 121.725401 83.752401) (width 0.3048) (layer B.Cu) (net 9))
 (segment (start 121.725401 83.752401) (end 121.352599 83.379599) (width 0.3048) (layer B.Cu) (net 9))
 (segment (start 121.352599 83.379599) (end 121.352599 81.982599) (width 0.3048) (layer B.Cu) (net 9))
 (segment (start 121.352599 81.982599) (end 120.717599 81.347599) (width 0.3048) (layer B.Cu) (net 9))
 (segment (start 117.984554 83.82) (end 111.125 83.82) (width 0.3048) (layer B.Cu) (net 9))
 (segment (start 120.717599 81.347599) (end 119.312401 81.347599) (width 0.3048) (layer B.Cu) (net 9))
 (segment (start 119.312401 81.347599) (end 118.677401 81.982599) (width 0.3048) (layer B.Cu) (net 9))
 (segment (start 118.677401 81.982599) (end 118.677401 83.127153) (width 0.3048) (layer B.Cu) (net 9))
 (segment (start 118.677401 83.127153) (end 117.984554 83.82) (width 0.3048) (layer B.Cu) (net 9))
 (segment (start 110.759 93.868) (end 111.125 94.234) (width 0.3048) (layer B.Cu) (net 1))
 (segment (start 108.839 93.868) (end 110.759 93.868) (width 0.3048) (layer B.Cu) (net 1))
 (segment (start 111.982999 93.376001) (end 111.125 94.234) (width 0.3048) (layer B.Cu) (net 1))
 (segment (start 112.208401 93.150599) (end 111.982999 93.376001) (width 0.3048) (layer B.Cu) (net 1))
 (segment (start 112.208401 91.351277) (end 112.208401 93.150599) (width 0.3048) (layer B.Cu) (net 1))
 (segment (start 112.672678 90.887) (end 112.208401 91.351277) (width 0.3048) (layer B.Cu) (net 1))
 (segment (start 113.607 90.887) (end 112.672678 90.887) (width 0.3048) (layer B.Cu) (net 1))
 (segment (start 111.125 91.6892) (end 111.125 91.694) (width 0.3048) (layer B.Cu) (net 10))
 (segment (start 112.5772 90.237) (end 111.125 91.6892) (width 0.3048) (layer B.Cu) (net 10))
 (segment (start 113.607 90.237) (end 112.5772 90.237) (width 0.3048) (layer B.Cu) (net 10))
 (segment (start 109.601 93.218) (end 111.125 91.694) (width 0.3048) (layer B.Cu) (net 10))
 (segment (start 108.839 93.218) (end 109.601 93.218) (width 0.3048) (layer B.Cu) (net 10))
 (segment (start 111.342 88.937) (end 111.125 89.154) (width 0.3048) (layer B.Cu) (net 11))
 (segment (start 113.607 88.937) (end 111.342 88.937) (width 0.3048) (layer B.Cu) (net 11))
 (segment (start 110.789 88.818) (end 111.125 89.154) (width 0.3048) (layer B.Cu) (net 11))
 (segment (start 108.957 88.818) (end 110.789 88.818) (width 0.3048) (layer B.Cu) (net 11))
 (segment (start 113.607 88.287) (end 112.5772 88.287) (width 0.3048) (layer B.Cu) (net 12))
 (segment (start 108.957 88.168) (end 109.728 88.168) (width 0.3048) (layer B.Cu) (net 12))
 (segment (start 109.728 88.168) (end 110.206 88.168) (width 0.3048) (layer B.Cu) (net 12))
 (segment (start 111.125 87.249) (end 111.125 86.36) (width 0.3048) (layer B.Cu) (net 12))
 (segment (start 110.617 87.757) (end 112.0472 87.757) (width 0.3048) (layer B.Cu) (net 12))
 (segment (start 112.5772 88.287) (end 112.0472 87.757) (width 0.3048) (layer B.Cu) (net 12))
 (segment (start 110.617 87.757) (end 111.125 87.249) (width 0.3048) (layer B.Cu) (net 12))
 (segment (start 110.206 88.168) (end 110.617 87.757) (width 0.3048) (layer B.Cu) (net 12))
 (segment (start 122.047 86.7768) (end 122.047 86.614) (width 0.3048) (layer B.Cu) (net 13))
 (segment (start 120.5368 88.287) (end 122.047 86.7768) (width 0.3048) (layer B.Cu) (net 13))
 (segment (start 119.507 88.287) (end 120.5368 88.287) (width 0.3048) (layer B.Cu) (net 13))
 (segment (start 122.383 86.95) (end 122.047 86.614) (width 0.3048) (layer B.Cu) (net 13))
 (segment (start 124.342 86.95) (end 122.383 86.95) (width 0.3048) (layer B.Cu) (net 13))
 (segment (start 121.83 88.937) (end 122.047 89.154) (width 0.3048) (layer B.Cu) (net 14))
 (segment (start 119.507 88.937) (end 121.83 88.937) (width 0.3048) (layer B.Cu) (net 14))
 (segment (start 122.047 88.9152) (end 122.047 89.154) (width 0.3048) (layer B.Cu) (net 14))
 (segment (start 123.3622 87.6) (end 122.047 88.9152) (width 0.3048) (layer B.Cu) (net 14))
 (segment (start 124.342 87.6) (end 123.3622 87.6) (width 0.3048) (layer B.Cu) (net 14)))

